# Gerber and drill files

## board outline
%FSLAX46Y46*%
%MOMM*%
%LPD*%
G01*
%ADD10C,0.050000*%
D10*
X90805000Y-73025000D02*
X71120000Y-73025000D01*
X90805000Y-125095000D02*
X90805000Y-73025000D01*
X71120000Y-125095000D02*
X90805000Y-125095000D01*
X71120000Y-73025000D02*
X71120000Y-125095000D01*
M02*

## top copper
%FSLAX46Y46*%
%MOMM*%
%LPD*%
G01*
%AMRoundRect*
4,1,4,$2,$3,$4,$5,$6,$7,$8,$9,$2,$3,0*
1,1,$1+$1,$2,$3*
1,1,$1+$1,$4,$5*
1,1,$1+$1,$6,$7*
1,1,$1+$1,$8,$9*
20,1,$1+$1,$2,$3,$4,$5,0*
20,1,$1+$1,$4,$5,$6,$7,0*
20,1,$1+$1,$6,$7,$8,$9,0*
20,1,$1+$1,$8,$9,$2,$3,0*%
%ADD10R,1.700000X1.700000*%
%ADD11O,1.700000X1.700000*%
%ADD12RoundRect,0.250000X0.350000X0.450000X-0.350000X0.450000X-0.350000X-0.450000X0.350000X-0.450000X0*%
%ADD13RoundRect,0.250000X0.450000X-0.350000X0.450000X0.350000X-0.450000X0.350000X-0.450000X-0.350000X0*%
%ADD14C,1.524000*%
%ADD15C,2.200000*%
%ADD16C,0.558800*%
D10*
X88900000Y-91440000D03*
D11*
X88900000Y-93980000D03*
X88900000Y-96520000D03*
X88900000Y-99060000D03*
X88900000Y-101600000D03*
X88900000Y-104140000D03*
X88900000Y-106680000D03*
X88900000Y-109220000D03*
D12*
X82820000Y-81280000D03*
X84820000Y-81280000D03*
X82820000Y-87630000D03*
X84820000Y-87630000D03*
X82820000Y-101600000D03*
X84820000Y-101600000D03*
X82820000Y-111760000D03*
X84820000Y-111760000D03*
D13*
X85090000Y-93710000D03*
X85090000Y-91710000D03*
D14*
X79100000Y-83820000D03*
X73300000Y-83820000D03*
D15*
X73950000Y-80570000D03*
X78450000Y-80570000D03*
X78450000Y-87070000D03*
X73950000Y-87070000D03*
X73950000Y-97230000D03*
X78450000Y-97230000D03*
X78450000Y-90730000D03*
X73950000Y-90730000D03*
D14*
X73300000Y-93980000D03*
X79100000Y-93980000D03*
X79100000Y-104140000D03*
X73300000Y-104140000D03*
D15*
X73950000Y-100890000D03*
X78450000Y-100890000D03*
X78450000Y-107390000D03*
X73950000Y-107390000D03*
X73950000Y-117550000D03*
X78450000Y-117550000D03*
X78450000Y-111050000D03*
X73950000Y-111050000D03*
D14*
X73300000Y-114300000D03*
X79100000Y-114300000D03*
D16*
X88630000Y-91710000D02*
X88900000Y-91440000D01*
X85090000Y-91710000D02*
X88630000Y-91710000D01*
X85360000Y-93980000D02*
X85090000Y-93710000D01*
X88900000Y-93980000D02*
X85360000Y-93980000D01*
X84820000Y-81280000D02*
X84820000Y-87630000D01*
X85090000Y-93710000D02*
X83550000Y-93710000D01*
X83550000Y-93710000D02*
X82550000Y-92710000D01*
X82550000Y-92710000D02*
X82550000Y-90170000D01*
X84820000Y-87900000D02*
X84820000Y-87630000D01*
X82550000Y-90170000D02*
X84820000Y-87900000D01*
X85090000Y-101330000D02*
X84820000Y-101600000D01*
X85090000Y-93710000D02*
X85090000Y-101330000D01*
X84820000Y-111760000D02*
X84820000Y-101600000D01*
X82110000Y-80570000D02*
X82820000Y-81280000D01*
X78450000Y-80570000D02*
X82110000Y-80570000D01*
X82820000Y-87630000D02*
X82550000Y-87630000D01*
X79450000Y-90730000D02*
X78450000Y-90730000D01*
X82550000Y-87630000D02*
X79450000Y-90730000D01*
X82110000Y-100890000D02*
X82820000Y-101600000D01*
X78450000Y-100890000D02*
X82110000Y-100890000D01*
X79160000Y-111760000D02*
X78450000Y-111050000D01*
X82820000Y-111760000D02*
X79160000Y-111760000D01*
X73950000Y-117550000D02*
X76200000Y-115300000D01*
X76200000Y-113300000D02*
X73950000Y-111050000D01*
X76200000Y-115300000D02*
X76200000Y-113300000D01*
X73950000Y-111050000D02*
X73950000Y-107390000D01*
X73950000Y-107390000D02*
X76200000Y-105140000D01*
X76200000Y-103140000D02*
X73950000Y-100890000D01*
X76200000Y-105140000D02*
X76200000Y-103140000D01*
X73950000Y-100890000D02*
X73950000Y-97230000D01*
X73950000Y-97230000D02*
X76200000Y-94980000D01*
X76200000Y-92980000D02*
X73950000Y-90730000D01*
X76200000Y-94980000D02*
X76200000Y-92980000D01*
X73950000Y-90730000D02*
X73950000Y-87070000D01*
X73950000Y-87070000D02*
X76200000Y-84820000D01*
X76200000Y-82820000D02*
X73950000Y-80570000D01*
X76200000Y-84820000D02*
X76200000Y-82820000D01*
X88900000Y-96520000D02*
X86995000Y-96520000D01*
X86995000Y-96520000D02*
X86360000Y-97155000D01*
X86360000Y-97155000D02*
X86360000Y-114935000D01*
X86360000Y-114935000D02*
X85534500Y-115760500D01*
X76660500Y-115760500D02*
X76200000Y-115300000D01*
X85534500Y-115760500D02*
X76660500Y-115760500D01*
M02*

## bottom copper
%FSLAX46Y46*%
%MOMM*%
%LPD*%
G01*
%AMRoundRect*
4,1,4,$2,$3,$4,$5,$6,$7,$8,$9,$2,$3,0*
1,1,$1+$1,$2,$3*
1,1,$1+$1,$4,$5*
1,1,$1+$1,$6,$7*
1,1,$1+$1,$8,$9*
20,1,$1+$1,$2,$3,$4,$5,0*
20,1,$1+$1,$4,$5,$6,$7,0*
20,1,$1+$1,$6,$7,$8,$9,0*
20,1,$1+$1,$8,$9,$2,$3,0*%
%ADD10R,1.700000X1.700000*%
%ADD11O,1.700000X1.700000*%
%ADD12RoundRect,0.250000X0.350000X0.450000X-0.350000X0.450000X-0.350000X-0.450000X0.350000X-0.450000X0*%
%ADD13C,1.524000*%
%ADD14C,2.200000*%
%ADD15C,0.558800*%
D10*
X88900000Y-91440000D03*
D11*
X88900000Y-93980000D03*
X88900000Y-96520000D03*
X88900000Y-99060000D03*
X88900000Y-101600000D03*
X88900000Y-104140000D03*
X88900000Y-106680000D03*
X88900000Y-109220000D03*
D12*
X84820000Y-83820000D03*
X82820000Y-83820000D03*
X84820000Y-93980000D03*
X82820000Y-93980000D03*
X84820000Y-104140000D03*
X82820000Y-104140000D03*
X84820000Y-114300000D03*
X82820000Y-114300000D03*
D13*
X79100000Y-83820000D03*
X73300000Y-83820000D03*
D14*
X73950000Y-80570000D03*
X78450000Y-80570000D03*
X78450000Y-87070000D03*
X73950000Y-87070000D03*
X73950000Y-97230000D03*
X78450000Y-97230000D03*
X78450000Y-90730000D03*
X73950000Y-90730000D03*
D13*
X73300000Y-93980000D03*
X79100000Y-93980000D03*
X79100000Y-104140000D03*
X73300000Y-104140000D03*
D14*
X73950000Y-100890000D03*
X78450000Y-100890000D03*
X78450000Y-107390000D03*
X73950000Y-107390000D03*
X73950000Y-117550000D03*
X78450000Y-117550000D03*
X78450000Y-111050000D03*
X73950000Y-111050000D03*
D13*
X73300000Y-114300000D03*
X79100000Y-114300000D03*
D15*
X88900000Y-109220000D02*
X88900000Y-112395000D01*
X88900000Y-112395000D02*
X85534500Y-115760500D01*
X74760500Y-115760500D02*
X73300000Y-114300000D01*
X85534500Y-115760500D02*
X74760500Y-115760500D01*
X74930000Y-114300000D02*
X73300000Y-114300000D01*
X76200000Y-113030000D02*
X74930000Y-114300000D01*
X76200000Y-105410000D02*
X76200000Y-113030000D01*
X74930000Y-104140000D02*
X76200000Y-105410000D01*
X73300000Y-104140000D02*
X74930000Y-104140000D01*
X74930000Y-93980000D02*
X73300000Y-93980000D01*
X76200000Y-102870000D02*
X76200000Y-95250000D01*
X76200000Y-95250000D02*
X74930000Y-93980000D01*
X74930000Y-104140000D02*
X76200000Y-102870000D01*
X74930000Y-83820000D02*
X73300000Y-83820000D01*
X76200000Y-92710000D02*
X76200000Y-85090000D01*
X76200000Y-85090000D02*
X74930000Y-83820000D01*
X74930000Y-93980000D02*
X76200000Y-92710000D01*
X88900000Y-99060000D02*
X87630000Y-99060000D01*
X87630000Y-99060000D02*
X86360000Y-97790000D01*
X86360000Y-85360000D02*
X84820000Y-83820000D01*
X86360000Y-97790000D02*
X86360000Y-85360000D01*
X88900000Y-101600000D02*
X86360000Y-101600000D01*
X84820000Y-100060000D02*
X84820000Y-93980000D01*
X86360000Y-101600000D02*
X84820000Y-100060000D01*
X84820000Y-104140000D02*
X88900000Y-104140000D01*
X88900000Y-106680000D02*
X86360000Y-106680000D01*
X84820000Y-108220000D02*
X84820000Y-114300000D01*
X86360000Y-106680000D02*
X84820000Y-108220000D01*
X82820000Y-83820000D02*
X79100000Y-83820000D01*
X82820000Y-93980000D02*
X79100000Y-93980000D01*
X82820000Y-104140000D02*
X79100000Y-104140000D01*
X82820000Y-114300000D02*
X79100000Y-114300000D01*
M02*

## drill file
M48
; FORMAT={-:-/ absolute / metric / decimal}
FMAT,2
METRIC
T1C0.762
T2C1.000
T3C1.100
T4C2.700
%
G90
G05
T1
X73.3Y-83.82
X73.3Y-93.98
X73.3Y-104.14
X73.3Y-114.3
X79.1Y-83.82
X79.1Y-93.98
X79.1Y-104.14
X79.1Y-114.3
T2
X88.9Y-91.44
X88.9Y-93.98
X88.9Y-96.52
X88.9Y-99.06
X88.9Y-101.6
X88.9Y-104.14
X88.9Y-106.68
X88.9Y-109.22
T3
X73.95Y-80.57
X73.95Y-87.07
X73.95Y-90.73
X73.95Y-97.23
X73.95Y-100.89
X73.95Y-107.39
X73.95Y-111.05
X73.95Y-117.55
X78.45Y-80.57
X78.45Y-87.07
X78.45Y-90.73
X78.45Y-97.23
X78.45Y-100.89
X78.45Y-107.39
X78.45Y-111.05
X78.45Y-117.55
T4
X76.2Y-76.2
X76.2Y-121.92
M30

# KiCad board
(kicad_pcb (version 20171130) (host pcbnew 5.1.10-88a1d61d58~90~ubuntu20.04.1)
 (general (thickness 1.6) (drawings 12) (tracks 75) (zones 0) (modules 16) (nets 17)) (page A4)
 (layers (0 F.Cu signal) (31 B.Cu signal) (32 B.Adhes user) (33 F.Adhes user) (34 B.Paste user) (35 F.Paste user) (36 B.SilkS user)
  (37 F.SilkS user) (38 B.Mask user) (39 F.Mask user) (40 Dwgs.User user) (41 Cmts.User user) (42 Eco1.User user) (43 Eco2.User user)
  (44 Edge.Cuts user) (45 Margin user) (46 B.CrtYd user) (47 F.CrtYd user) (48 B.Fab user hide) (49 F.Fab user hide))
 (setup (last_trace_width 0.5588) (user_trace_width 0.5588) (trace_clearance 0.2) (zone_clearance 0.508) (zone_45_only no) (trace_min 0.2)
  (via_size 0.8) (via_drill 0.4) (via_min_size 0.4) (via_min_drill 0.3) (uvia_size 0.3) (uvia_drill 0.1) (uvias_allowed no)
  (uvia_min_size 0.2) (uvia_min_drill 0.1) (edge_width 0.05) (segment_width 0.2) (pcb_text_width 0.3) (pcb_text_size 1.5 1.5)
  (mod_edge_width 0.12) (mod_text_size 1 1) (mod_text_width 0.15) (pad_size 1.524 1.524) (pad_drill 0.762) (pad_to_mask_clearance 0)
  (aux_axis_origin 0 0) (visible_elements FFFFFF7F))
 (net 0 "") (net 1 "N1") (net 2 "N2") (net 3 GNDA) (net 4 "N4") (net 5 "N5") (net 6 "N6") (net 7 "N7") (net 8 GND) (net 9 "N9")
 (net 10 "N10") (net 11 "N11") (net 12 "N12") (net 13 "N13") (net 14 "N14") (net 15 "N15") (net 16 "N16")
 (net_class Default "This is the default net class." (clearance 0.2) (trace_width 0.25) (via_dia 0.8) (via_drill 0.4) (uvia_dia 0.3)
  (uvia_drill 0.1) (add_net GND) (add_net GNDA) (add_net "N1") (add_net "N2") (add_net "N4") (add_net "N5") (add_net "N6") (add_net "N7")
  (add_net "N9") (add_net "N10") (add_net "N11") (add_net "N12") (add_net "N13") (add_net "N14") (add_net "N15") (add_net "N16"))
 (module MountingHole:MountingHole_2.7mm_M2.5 (layer F.Cu) (at 76.2 76.2)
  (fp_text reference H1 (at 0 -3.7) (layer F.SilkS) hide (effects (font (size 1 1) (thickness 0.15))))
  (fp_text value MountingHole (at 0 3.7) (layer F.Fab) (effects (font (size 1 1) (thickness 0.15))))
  (pad 1 np_thru_hole circle (at 0 0) (size 2.7 2.7) (drill 2.7) (layers *.Cu *.Mask)))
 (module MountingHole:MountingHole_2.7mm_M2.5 (layer F.Cu) (at 76.2 121.92)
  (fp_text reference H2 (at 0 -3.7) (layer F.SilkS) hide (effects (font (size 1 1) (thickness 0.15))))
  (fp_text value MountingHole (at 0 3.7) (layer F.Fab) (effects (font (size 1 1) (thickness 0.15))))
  (pad 1 np_thru_hole circle (at 0 0) (size 2.7 2.7) (drill 2.7) (layers *.Cu *.Mask)))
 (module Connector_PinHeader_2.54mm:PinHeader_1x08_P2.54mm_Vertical (layer F.Cu) (at 88.9 91.44)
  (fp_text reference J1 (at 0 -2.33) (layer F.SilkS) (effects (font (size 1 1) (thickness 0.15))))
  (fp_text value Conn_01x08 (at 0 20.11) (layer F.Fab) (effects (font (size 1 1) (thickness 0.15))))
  (pad 1 thru_hole rect (at 0 0) (size 1.7 1.7) (drill 1) (layers *.Cu *.Mask) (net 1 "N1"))
  (pad 2 thru_hole oval (at 0 2.54) (size 1.7 1.7) (drill 1) (layers *.Cu *.Mask) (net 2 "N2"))
  (pad 3 thru_hole oval (at 0 5.08) (size 1.7 1.7) (drill 1) (layers *.Cu *.Mask) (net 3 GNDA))
  (pad 4 thru_hole oval (at 0 7.62) (size 1.7 1.7) (drill 1) (layers *.Cu *.Mask) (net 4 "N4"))
  (pad 5 thru_hole oval (at 0 10.16) (size 1.7 1.7) (drill 1) (layers *.Cu *.Mask) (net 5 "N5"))
  (pad 6 thru_hole oval (at 0 12.7) (size 1.7 1.7) (drill 1) (layers *.Cu *.Mask) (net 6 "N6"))
  (pad 7 thru_hole oval (at 0 15.24) (size 1.7 1.7) (drill 1) (layers *.Cu *.Mask) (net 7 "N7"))
  (pad 8 thru_hole oval (at 0 17.78) (size 1.7 1.7) (drill 1) (layers *.Cu *.Mask) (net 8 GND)))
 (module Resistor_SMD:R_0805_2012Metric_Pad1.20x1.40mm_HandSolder (layer B.Cu) (at 83.82 83.82 180)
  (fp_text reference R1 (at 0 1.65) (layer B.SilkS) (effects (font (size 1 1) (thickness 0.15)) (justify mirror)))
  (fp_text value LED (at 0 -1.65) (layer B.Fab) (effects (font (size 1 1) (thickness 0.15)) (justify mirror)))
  (pad 1 smd roundrect (at -1 0 180) (size 1.2 1.4) (layers B.Cu B.Paste B.Mask) (roundrect_rratio 0.208333) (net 4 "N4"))
  (pad 2 smd roundrect (at 1 0 180) (size 1.2 1.4) (layers B.Cu B.Paste B.Mask) (roundrect_rratio 0.208333) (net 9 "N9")))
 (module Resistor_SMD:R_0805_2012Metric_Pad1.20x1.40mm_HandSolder (layer B.Cu) (at 83.82 93.98 180)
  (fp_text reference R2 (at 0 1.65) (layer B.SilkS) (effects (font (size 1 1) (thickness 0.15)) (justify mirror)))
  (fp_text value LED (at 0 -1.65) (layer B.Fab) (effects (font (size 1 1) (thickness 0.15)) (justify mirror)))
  (pad 1 smd roundrect (at -1 0 180) (size 1.2 1.4) (layers B.Cu B.Paste B.Mask) (roundrect_rratio 0.208333) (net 5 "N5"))
  (pad 2 smd roundrect (at 1 0 180) (size 1.2 1.4) (layers B.Cu B.Paste B.Mask) (roundrect_rratio 0.208333) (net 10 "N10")))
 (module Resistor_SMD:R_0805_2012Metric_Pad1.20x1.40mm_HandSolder (layer B.Cu) (at 83.82 104.14 180)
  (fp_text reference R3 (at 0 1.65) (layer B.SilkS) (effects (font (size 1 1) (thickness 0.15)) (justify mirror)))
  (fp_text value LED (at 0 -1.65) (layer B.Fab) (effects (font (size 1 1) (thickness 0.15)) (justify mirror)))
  (pad 1 smd roundrect (at -1 0 180) (size 1.2 1.4) (layers B.Cu B.Paste B.Mask) (roundrect_rratio 0.208333) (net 6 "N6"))
  (pad 2 smd roundrect (at 1 0 180) (size 1.2 1.4) (layers B.Cu B.Paste B.Mask) (roundrect_rratio 0.208333) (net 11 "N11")))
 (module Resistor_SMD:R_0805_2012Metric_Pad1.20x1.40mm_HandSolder (layer B.Cu) (at 83.82 114.3 180)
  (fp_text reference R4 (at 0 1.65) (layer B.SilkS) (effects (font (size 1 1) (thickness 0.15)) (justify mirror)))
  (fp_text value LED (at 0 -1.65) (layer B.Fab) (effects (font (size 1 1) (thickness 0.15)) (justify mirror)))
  (pad 1 smd roundrect (at -1 0 180) (size 1.2 1.4) (layers B.Cu B.Paste B.Mask) (roundrect_rratio 0.208333) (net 7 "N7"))
  (pad 2 smd roundrect (at 1 0 180) (size 1.2 1.4) (layers B.Cu B.Paste B.Mask) (roundrect_rratio 0.208333) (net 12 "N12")))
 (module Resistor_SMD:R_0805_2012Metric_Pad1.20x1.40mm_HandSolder (layer F.Cu) (at 83.82 81.28 180)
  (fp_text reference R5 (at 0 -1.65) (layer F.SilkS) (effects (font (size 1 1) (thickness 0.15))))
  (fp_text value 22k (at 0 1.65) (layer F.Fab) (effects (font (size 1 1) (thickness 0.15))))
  (pad 2 smd roundrect (at 1 0 180) (size 1.2 1.4) (layers F.Cu F.Paste F.Mask) (roundrect_rratio 0.208333) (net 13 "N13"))
  (pad 1 smd roundrect (at -1 0 180) (size 1.2 1.4) (layers F.Cu F.Paste F.Mask) (roundrect_rratio 0.208333) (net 2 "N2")))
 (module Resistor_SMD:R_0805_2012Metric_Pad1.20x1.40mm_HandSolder (layer F.Cu) (at 83.82 87.63 180)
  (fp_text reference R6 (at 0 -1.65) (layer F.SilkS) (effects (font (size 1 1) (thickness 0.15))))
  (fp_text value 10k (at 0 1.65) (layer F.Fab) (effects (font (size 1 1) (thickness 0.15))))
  (pad 2 smd roundrect (at 1 0 180) (size 1.2 1.4) (layers F.Cu F.Paste F.Mask) (roundrect_rratio 0.208333) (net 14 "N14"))
  (pad 1 smd roundrect (at -1 0 180) (size 1.2 1.4) (layers F.Cu F.Paste F.Mask) (roundrect_rratio 0.208333) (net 2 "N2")))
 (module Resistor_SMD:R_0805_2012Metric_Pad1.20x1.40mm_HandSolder (layer F.Cu) (at 83.82 101.6 180)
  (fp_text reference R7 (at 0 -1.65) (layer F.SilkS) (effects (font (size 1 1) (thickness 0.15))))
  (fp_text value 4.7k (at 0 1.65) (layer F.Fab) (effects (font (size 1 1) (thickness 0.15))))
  (pad 2 smd roundrect (at 1 0 180) (size 1.2 1.4) (layers F.Cu F.Paste F.Mask) (roundrect_rratio 0.208333) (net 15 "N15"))
  (pad 1 smd roundrect (at -1 0 180) (size 1.2 1.4) (layers F.Cu F.Paste F.Mask) (roundrect_rratio 0.208333) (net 2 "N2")))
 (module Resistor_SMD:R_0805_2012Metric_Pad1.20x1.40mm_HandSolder (layer F.Cu) (at 83.82 111.76 180)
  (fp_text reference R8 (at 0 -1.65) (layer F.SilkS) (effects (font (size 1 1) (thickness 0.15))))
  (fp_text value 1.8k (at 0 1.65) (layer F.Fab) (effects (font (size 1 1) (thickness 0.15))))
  (pad 2 smd roundrect (at 1 0 180) (size 1.2 1.4) (layers F.Cu F.Paste F.Mask) (roundrect_rratio 0.208333) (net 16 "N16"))
  (pad 1 smd roundrect (at -1 0 180) (size 1.2 1.4) (layers F.Cu F.Paste F.Mask) (roundrect_rratio 0.208333) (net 2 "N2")))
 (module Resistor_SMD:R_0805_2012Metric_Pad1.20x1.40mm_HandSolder (layer F.Cu) (at 85.09 92.71 90)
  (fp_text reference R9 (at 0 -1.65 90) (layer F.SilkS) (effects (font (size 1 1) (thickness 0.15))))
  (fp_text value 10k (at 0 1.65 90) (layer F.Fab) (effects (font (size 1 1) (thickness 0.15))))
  (pad 1 smd roundrect (at -1 0 90) (size 1.2 1.4) (layers F.Cu F.Paste F.Mask) (roundrect_rratio 0.208333) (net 2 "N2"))
  (pad 2 smd roundrect (at 1 0 90) (size 1.2 1.4) (layers F.Cu F.Paste F.Mask) (roundrect_rratio 0.208333) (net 1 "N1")))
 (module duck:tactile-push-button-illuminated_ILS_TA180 (layer F.Cu) (at 76.2 83.82 270)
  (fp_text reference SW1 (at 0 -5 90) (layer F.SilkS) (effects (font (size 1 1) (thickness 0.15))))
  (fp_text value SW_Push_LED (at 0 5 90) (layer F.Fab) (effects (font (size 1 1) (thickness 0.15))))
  (pad 4 thru_hole circle (at 0 -2.9 270) (size 1.524 1.524) (drill 0.762) (layers *.Cu *.Mask) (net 9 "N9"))
  (pad 3 thru_hole circle (at 0 2.9 270) (size 1.524 1.524) (drill 0.762) (layers *.Cu *.Mask) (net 8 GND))
  (pad 1 thru_hole circle (at -3.25 2.25 270) (size 2.2 2.2) (drill 1.1) (layers *.Cu *.Mask) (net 3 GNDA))
  (pad 2 thru_hole circle (at -3.25 -2.25 270) (size 2.2 2.2) (drill 1.1) (layers *.Cu *.Mask) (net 13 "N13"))
  (pad 2 thru_hole circle (at 3.25 -2.25 270) (size 2.2 2.2) (drill 1.1) (layers *.Cu *.Mask) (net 13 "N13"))
  (pad 1 thru_hole circle (at 3.25 2.25 270) (size 2.2 2.2) (drill 1.1) (layers *.Cu *.Mask) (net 3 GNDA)))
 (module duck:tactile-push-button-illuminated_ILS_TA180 (layer F.Cu) (at 76.2 93.98 270)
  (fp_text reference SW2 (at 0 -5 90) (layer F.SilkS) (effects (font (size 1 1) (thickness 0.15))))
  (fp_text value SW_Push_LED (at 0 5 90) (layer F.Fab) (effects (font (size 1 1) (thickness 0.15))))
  (pad 1 thru_hole circle (at 3.25 2.25 270) (size 2.2 2.2) (drill 1.1) (layers *.Cu *.Mask) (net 3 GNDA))
  (pad 2 thru_hole circle (at 3.25 -2.25 270) (size 2.2 2.2) (drill 1.1) (layers *.Cu *.Mask) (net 14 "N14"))
  (pad 2 thru_hole circle (at -3.25 -2.25 270) (size 2.2 2.2) (drill 1.1) (layers *.Cu *.Mask) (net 14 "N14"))
  (pad 1 thru_hole circle (at -3.25 2.25 270) (size 2.2 2.2) (drill 1.1) (layers *.Cu *.Mask) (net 3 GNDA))
  (pad 3 thru_hole circle (at 0 2.9 270) (size 1.524 1.524) (drill 0.762) (layers *.Cu *.Mask) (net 8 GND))
  (pad 4 thru_hole circle (at 0 -2.9 270) (size 1.524 1.524) (drill 0.762) (layers *.Cu *.Mask) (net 10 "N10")))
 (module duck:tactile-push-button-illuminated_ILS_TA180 (layer F.Cu) (at 76.2 104.14 270)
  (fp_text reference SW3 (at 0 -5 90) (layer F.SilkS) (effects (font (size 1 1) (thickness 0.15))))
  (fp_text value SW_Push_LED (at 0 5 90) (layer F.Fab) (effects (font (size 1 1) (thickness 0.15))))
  (pad 4 thru_hole circle (at 0 -2.9 270) (size 1.524 1.524) (drill 0.762) (layers *.Cu *.Mask) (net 11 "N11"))
  (pad 3 thru_hole circle (at 0 2.9 270) (size 1.524 1.524) (drill 0.762) (layers *.Cu *.Mask) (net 8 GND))
  (pad 1 thru_hole circle (at -3.25 2.25 270) (size 2.2 2.2) (drill 1.1) (layers *.Cu *.Mask) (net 3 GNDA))
  (pad 2 thru_hole circle (at -3.25 -2.25 270) (size 2.2 2.2) (drill 1.1) (layers *.Cu *.Mask) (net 15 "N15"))
  (pad 2 thru_hole circle (at 3.25 -2.25 270) (size 2.2 2.2) (drill 1.1) (layers *.Cu *.Mask) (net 15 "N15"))
  (pad 1 thru_hole circle (at 3.25 2.25 270) (size 2.2 2.2) (drill 1.1) (layers *.Cu *.Mask) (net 3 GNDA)))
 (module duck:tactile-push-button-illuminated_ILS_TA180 (layer F.Cu) (at 76.2 114.3 270)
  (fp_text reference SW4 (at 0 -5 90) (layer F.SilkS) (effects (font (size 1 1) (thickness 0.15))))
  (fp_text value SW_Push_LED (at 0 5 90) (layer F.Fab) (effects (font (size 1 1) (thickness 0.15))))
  (pad 1 thru_hole circle (at 3.25 2.25 270) (size 2.2 2.2) (drill 1.1) (layers *.Cu *.Mask) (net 3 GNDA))
  (pad 2 thru_hole circle (at 3.25 -2.25 270) (size 2.2 2.2) (drill 1.1) (layers *.Cu *.Mask) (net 16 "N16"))
  (pad 2 thru_hole circle (at -3.25 -2.25 270) (size 2.2 2.2) (drill 1.1) (layers *.Cu *.Mask) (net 16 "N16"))
  (pad 1 thru_hole circle (at -3.25 2.25 270) (size 2.2 2.2) (drill 1.1) (layers *.Cu *.Mask) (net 3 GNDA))
  (pad 3 thru_hole circle (at 0 2.9 270) (size 1.524 1.524) (drill 0.762) (layers *.Cu *.Mask) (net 8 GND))
  (pad 4 thru_hole circle (at 0 -2.9 270) (size 1.524 1.524) (drill 0.762) (layers *.Cu *.Mask) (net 12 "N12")))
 (gr_line (start 90.805 73.025) (end 71.12 73.025) (layer Edge.Cuts) (width 0.05))
 (gr_line (start 90.805 125.095) (end 90.805 73.025) (layer Edge.Cuts) (width 0.05))
 (gr_line (start 71.12 125.095) (end 90.805 125.095) (layer Edge.Cuts) (width 0.05))
 (gr_line (start 71.12 73.025) (end 71.12 125.095) (layer Edge.Cuts) (width 0.05))
 (segment (start 88.63 91.71) (end 88.9 91.44) (width 0.5588) (layer F.Cu) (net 1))
 (segment (start 85.09 91.71) (end 88.63 91.71) (width 0.5588) (layer F.Cu) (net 1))
 (segment (start 85.36 93.98) (end 85.09 93.71) (width 0.5588) (layer F.Cu) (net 2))
 (segment (start 88.9 93.98) (end 85.36 93.98) (width 0.5588) (layer F.Cu) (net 2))
 (segment (start 84.82 81.28) (end 84.82 87.63) (width 0.5588) (layer F.Cu) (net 2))
 (segment (start 85.09 93.71) (end 83.55 93.71) (width 0.5588) (layer F.Cu) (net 2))
 (segment (start 83.55 93.71) (end 82.55 92.71) (width 0.5588) (layer F.Cu) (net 2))
 (segment (start 82.55 92.71) (end 82.55 90.17) (width 0.5588) (layer F.Cu) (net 2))
 (segment (start 84.82 87.9) (end 84.82 87.63) (width 0.5588) (layer F.Cu) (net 2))
 (segment (start 82.55 90.17) (end 84.82 87.9) (width 0.5588) (layer F.Cu) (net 2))
 (segment (start 85.09 101.33) (end 84.82 101.6) (width 0.5588) (layer F.Cu) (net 2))
 (segment (start 85.09 93.71) (end 85.09 101.33) (width 0.5588) (layer F.Cu) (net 2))
 (segment (start 84.82 111.76) (end 84.82 101.6) (width 0.5588) (layer F.Cu) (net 2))
 (segment (start 88.9 109.22) (end 88.9 112.395) (width 0.5588) (layer B.Cu) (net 8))
 (segment (start 88.9 112.395) (end 85.5345 115.7605) (width 0.5588) (layer B.Cu) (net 8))
 (segment (start 74.7605 115.7605) (end 73.3 114.3) (width 0.5588) (layer B.Cu) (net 8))
 (segment (start 85.5345 115.7605) (end 74.7605 115.7605) (width 0.5588) (layer B.Cu) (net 8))
 (segment (start 74.93 114.3) (end 73.3 114.3) (width 0.5588) (layer B.Cu) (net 8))
 (segment (start 76.2 113.03) (end 74.93 114.3) (width 0.5588) (layer B.Cu) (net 8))
 (segment (start 76.2 105.41) (end 76.2 113.03) (width 0.5588) (layer B.Cu) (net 8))
 (segment (start 74.93 104.14) (end 76.2 105.41) (width 0.5588) (layer B.Cu) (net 8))
 (segment (start 73.3 104.14) (end 74.93 104.14) (width 0.5588) (layer B.Cu) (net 8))
 (segment (start 74.93 93.98) (end 73.3 93.98) (width 0.5588) (layer B.Cu) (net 8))
 (segment (start 76.2 102.87) (end 76.2 95.25) (width 0.5588) (layer B.Cu) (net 8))
 (segment (start 76.2 95.25) (end 74.93 93.98) (width 0.5588) (layer B.Cu) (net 8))
 (segment (start 74.93 104.14) (end 76.2 102.87) (width 0.5588) (layer B.Cu) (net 8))
 (segment (start 74.93 83.82) (end 73.3 83.82) (width 0.5588) (layer B.Cu) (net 8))
 (segment (start 76.2 92.71) (end 76.2 85.09) (width 0.5588) (layer B.Cu) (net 8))
 (segment (start 76.2 85.09) (end 74.93 83.82) (width 0.5588) (layer B.Cu) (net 8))
 (segment (start 74.93 93.98) (end 76.2 92.71) (width 0.5588) (layer B.Cu) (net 8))
 (segment (start 88.9 99.06) (end 87.63 99.06) (width 0.5588) (layer B.Cu) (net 4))
 (segment (start 87.63 99.06) (end 86.36 97.79) (width 0.5588) (layer B.Cu) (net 4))
 (segment (start 86.36 85.36) (end 84.82 83.82) (width 0.5588) (layer B.Cu) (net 4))
 (segment (start 86.36 97.79) (end 86.36 85.36) (width 0.5588) (layer B.Cu) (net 4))
 (segment (start 88.9 101.6) (end 86.36 101.6) (width 0.5588) (layer B.Cu) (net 5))
 (segment (start 84.82 100.06) (end 84.82 93.98) (width 0.5588) (layer B.Cu) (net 5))
 (segment (start 86.36 101.6) (end 84.82 100.06) (width 0.5588) (layer B.Cu) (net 5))
 (segment (start 84.82 104.14) (end 88.9 104.14) (width 0.5588) (layer B.Cu) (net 6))
 (segment (start 88.9 106.68) (end 86.36 106.68) (width 0.5588) (layer B.Cu) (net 7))
 (segment (start 84.82 108.22) (end 84.82 114.3) (width 0.5588) (layer B.Cu) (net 7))
 (segment (start 86.36 106.68) (end 84.82 108.22) (width 0.5588) (layer B.Cu) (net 7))
 (segment (start 82.82 83.82) (end 79.1 83.82) (width 0.5588) (layer B.Cu) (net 9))
 (segment (start 82.82 93.98) (end 79.1 93.98) (width 0.5588) (layer B.Cu) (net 10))
 (segment (start 82.82 104.14) (end 79.1 104.14) (width 0.5588) (layer B.Cu) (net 11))
 (segment (start 82.82 114.3) (end 79.1 114.3) (width 0.5588) (layer B.Cu) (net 12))
 (segment (start 82.11 80.57) (end 82.82 81.28) (width 0.5588) (layer F.Cu) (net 13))
 (segment (start 78.45 80.57) (end 82.11 80.57) (width 0.5588) (layer F.Cu) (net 13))
 (segment (start 82.82 87.63) (end 82.55 87.63) (width 0.5588) (layer F.Cu) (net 14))
 (segment (start 79.45 90.73) (end 78.45 90.73) (width 0.5588) (layer F.Cu) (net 14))
 (segment (start 82.55 87.63) (end 79.45 90.73) (width 0.5588) (layer F.Cu) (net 14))
 (segment (start 82.11 100.89) (end 82.82 101.6) (width 0.5588) (layer F.Cu) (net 15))
 (segment (start 78.45 100.89) (end 82.11 100.89) (width 0.5588) (layer F.Cu) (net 15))
 (segment (start 79.16 111.76) (end 78.45 111.05) (width 0.5588) (layer F.Cu) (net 16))
 (segment (start 82.82 111.76) (end 79.16 111.76) (width 0.5588) (layer F.Cu) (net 16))
 (segment (start 73.95 117.55) (end 76.2 115.3) (width 0.5588) (layer F.Cu) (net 3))
 (segment (start 76.2 113.3) (end 73.95 111.05) (width 0.5588) (layer F.Cu) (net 3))
 (segment (start 76.2 115.3) (end 76.2 113.3) (width 0.5588) (layer F.Cu) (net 3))
 (segment (start 73.95 111.05) (end 73.95 107.39) (width 0.5588) (layer F.Cu) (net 3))
 (segment (start 73.95 107.39) (end 76.2 105.14) (width 0.5588) (layer F.Cu) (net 3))
 (segment (start 76.2 103.14) (end 73.95 100.89) (width 0.5588) (layer F.Cu) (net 3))
 (segment (start 76.2 105.14) (end 76.2 103.14) (width 0.5588) (layer F.Cu) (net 3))
 (segment (start 73.95 100.89) (end 73.95 97.23) (width 0.5588) (layer F.Cu) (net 3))
 (segment (start 73.95 97.23) (end 76.2 94.98) (width 0.5588) (layer F.Cu) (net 3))
 (segment (start 76.2 92.98) (end 73.95 90.73) (width 0.5588) (layer F.Cu) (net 3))
 (segment (start 76.2 94.98) (end 76.2 92.98) (width 0.5588) (layer F.Cu) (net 3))
 (segment (start 73.95 90.73) (end 73.95 87.07) (width 0.5588) (layer F.Cu) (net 3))
 (segment (start 73.95 87.07) (end 76.2 84.82) (width 0.5588) (layer F.Cu) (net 3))
 (segment (start 76.2 82.82) (end 73.95 80.57) (width 0.5588) (layer F.Cu) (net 3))
 (segment (start 76.2 84.82) (end 76.2 82.82) (width 0.5588) (layer F.Cu) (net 3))
 (segment (start 88.9 96.52) (end 86.995 96.52) (width 0.5588) (layer F.Cu) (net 3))
 (segment (start 86.995 96.52) (end 86.36 97.155) (width 0.5588) (layer F.Cu) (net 3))
 (segment (start 86.36 97.155) (end 86.36 114.935) (width 0.5588) (layer F.Cu) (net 3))
 (segment (start 86.36 114.935) (end 85.5345 115.7605) (width 0.5588) (layer F.Cu) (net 3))
 (segment (start 76.6605 115.7605) (end 76.2 115.3) (width 0.5588) (layer F.Cu) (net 3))
 (segment (start 85.5345 115.7605) (end 76.6605 115.7605) (width 0.5588) (layer F.Cu) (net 3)))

